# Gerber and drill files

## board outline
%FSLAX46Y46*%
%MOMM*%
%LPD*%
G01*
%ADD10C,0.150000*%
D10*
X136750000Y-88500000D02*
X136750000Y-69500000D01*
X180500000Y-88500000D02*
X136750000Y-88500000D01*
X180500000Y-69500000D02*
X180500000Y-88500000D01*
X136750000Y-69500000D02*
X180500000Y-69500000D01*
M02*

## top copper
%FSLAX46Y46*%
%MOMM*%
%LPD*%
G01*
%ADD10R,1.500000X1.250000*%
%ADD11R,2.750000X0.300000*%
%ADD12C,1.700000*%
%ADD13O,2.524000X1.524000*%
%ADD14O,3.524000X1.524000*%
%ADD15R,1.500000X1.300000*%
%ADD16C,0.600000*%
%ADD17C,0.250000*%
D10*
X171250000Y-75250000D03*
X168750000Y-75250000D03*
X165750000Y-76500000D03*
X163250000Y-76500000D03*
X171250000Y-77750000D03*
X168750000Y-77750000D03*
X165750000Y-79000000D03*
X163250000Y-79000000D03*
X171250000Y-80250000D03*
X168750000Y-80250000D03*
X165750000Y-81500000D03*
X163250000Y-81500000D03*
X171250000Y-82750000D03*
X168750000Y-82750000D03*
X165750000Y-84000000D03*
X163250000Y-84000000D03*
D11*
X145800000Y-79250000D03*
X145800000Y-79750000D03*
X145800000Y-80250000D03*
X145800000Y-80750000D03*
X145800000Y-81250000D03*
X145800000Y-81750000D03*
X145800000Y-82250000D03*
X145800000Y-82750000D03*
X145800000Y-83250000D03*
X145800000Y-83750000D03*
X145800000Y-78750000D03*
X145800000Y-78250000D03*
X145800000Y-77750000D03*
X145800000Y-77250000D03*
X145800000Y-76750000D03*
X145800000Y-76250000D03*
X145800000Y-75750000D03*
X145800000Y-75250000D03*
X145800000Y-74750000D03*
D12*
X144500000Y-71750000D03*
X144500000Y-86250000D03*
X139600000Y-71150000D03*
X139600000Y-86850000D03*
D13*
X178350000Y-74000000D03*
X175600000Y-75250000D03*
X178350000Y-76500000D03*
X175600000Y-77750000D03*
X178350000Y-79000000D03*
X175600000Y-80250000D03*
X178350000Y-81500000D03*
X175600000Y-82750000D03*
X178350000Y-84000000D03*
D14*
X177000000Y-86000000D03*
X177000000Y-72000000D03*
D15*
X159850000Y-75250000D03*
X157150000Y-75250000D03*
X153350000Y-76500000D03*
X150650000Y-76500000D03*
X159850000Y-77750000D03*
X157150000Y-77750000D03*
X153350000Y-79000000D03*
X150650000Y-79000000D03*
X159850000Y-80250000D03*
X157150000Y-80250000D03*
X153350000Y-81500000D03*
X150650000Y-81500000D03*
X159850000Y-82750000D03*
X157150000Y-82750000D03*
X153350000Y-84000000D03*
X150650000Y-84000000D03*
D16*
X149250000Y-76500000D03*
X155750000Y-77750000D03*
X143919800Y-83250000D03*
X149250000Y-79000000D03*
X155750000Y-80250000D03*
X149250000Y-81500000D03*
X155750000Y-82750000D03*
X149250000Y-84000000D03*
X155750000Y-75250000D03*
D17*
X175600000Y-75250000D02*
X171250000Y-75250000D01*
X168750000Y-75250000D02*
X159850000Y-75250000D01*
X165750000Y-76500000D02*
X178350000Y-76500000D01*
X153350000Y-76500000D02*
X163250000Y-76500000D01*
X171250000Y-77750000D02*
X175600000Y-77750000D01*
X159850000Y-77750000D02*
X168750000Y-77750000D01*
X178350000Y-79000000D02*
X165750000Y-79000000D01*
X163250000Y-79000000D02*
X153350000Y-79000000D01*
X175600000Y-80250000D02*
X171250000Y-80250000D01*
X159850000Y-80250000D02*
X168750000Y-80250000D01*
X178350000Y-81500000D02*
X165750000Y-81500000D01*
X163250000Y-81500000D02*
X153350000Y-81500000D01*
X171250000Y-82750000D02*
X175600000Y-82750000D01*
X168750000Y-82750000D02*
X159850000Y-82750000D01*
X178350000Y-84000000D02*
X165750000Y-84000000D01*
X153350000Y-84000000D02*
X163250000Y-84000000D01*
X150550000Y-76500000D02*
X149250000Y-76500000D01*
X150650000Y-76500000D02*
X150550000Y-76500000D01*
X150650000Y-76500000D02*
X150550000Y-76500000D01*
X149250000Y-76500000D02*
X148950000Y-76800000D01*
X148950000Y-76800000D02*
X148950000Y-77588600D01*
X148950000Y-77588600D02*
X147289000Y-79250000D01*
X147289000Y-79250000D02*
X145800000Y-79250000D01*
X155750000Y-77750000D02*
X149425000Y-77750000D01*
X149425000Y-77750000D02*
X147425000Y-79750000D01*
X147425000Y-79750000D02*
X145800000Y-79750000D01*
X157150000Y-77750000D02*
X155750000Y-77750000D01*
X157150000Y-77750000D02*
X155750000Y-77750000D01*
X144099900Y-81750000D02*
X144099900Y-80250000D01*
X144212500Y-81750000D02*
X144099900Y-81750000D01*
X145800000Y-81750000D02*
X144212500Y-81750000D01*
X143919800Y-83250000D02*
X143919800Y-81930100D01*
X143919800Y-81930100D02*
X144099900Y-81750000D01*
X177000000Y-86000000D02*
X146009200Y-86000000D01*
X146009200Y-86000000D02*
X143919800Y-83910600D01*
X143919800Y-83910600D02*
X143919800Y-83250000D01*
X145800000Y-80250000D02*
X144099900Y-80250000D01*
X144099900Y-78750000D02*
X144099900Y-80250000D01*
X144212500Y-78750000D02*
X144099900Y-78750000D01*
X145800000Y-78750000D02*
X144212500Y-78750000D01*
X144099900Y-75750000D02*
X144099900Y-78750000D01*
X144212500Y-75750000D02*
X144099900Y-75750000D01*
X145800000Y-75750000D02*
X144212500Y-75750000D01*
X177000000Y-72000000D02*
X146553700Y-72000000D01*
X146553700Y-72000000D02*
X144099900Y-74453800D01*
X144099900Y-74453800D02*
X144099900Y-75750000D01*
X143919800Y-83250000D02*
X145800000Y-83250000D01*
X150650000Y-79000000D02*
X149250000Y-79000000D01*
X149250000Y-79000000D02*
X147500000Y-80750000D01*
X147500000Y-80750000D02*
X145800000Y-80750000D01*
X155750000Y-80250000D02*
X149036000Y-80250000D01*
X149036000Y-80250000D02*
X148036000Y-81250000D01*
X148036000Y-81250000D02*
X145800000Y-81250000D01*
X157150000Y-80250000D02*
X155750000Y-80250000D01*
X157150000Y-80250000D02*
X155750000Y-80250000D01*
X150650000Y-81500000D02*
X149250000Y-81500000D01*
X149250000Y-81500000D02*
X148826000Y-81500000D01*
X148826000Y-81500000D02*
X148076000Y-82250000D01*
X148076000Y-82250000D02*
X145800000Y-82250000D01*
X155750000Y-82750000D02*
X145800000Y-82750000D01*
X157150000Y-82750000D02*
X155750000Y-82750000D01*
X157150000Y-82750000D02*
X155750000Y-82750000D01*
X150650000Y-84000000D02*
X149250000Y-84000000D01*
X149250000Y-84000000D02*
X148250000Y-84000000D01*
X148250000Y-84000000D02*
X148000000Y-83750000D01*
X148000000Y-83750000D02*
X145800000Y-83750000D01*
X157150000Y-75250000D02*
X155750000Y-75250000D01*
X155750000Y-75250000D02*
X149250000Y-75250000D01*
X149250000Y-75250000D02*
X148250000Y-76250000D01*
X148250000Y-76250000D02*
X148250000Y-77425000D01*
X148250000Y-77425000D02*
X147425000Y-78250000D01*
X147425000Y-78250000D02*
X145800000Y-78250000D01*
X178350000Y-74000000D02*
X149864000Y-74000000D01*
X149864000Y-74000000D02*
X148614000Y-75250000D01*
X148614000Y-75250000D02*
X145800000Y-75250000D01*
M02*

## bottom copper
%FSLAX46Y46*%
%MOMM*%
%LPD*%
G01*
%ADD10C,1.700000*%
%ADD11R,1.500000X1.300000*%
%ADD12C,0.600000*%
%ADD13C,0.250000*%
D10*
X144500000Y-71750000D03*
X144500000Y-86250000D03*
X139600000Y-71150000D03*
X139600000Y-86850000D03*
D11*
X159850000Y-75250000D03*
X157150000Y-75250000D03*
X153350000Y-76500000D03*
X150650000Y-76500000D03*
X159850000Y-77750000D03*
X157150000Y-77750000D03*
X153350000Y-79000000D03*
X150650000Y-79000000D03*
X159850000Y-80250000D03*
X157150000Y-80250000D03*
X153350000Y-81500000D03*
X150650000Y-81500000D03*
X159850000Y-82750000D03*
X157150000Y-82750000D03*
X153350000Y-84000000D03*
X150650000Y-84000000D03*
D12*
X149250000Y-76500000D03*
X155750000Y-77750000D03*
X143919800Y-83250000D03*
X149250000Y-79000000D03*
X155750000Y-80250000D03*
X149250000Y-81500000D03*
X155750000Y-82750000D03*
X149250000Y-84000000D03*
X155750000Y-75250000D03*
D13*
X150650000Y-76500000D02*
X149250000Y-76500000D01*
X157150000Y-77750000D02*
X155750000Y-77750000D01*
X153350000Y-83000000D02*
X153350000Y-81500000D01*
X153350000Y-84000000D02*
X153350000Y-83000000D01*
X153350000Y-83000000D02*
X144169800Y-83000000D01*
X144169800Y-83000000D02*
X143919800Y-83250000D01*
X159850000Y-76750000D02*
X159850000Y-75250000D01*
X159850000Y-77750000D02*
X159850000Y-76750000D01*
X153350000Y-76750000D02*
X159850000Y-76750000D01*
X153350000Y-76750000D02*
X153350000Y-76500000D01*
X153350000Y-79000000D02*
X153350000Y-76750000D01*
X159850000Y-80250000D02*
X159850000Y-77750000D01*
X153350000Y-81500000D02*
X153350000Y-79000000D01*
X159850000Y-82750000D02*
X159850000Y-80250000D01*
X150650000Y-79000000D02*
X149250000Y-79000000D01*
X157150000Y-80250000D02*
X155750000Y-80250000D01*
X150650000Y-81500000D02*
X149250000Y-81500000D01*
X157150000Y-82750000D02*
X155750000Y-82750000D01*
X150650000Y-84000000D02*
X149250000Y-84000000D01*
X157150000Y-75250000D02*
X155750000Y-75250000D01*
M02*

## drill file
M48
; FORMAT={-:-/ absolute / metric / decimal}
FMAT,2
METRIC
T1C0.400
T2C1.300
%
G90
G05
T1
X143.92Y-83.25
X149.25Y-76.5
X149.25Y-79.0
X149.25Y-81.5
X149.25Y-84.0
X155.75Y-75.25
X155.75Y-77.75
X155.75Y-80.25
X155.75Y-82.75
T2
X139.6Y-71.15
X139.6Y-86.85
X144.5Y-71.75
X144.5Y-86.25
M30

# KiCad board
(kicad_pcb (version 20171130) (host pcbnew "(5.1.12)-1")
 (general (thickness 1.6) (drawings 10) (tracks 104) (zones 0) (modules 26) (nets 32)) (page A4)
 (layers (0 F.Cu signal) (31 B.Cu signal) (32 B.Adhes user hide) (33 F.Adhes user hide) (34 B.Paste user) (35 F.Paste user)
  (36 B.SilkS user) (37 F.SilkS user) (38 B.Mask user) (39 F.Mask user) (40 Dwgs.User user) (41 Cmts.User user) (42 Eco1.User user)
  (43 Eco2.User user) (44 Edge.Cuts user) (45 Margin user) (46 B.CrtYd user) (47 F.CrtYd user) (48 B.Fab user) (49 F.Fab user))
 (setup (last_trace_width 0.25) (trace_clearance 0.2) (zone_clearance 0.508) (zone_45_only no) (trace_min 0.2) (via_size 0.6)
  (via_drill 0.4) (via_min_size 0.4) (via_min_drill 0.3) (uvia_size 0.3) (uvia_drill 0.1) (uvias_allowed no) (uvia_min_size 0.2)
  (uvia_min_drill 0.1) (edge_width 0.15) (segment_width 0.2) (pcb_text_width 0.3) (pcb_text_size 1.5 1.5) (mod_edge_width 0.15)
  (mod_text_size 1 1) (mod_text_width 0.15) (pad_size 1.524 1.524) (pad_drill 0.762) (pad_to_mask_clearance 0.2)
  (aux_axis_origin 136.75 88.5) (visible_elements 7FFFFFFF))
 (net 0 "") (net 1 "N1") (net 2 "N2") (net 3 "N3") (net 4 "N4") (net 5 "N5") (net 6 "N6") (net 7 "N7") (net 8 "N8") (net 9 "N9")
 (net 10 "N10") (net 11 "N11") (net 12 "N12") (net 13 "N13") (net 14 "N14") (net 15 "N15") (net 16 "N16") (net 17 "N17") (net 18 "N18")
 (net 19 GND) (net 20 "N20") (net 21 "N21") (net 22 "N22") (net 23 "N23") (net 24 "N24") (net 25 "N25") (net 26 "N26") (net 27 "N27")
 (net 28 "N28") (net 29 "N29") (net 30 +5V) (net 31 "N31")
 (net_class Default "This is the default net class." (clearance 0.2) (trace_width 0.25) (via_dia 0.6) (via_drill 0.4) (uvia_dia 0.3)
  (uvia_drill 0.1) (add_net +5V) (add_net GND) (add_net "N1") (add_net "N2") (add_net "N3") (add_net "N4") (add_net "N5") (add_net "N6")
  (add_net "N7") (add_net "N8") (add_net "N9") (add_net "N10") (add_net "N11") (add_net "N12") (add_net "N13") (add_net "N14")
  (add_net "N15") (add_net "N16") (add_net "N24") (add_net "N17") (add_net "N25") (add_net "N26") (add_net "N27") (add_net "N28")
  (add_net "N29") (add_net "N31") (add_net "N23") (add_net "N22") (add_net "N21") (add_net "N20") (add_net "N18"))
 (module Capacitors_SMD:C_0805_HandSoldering (layer F.Cu) (at 170 75.25 180)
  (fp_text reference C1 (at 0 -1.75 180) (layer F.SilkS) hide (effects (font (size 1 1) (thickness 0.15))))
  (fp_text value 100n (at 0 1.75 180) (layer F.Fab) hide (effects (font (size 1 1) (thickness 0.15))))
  (pad 1 smd rect (at -1.25 0 180) (size 1.5 1.25) (layers F.Cu F.Paste F.Mask) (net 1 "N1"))
  (pad 2 smd rect (at 1.25 0 180) (size 1.5 1.25) (layers F.Cu F.Paste F.Mask) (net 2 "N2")))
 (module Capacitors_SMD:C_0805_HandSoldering (layer F.Cu) (at 164.5 76.5 180)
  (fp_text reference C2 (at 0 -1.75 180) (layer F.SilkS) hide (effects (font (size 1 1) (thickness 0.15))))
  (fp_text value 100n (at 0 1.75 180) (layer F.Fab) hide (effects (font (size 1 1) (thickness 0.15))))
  (pad 1 smd rect (at -1.25 0 180) (size 1.5 1.25) (layers F.Cu F.Paste F.Mask) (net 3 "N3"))
  (pad 2 smd rect (at 1.25 0 180) (size 1.5 1.25) (layers F.Cu F.Paste F.Mask) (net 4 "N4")))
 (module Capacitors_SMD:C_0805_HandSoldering (layer F.Cu) (at 170 77.75 180)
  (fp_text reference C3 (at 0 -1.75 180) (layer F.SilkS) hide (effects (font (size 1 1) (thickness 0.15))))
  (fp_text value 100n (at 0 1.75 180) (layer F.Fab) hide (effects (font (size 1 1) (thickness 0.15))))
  (pad 1 smd rect (at -1.25 0 180) (size 1.5 1.25) (layers F.Cu F.Paste F.Mask) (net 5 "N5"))
  (pad 2 smd rect (at 1.25 0 180) (size 1.5 1.25) (layers F.Cu F.Paste F.Mask) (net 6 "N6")))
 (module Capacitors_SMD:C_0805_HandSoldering (layer F.Cu) (at 164.5 79 180)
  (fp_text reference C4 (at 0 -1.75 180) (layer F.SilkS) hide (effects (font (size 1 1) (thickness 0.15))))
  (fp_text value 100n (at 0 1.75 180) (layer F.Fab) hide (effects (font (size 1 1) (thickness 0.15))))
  (pad 1 smd rect (at -1.25 0 180) (size 1.5 1.25) (layers F.Cu F.Paste F.Mask) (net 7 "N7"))
  (pad 2 smd rect (at 1.25 0 180) (size 1.5 1.25) (layers F.Cu F.Paste F.Mask) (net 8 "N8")))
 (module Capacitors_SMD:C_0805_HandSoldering (layer F.Cu) (at 170 80.25 180)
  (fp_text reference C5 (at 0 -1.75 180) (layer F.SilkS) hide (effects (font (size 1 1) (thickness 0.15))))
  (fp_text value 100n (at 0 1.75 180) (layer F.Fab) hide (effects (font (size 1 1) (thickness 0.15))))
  (pad 1 smd rect (at -1.25 0 180) (size 1.5 1.25) (layers F.Cu F.Paste F.Mask) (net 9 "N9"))
  (pad 2 smd rect (at 1.25 0 180) (size 1.5 1.25) (layers F.Cu F.Paste F.Mask) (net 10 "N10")))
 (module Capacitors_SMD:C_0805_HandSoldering (layer F.Cu) (at 164.5 81.5 180)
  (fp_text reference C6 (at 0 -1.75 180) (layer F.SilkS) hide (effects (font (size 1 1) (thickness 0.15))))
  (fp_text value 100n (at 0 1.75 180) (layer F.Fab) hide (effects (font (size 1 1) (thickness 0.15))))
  (pad 1 smd rect (at -1.25 0 180) (size 1.5 1.25) (layers F.Cu F.Paste F.Mask) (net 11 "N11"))
  (pad 2 smd rect (at 1.25 0 180) (size 1.5 1.25) (layers F.Cu F.Paste F.Mask) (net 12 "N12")))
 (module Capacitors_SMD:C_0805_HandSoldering (layer F.Cu) (at 170 82.75 180)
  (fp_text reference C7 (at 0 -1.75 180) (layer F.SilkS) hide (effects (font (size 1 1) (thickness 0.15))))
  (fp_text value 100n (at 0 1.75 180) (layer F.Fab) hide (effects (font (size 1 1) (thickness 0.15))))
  (pad 1 smd rect (at -1.25 0 180) (size 1.5 1.25) (layers F.Cu F.Paste F.Mask) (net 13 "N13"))
  (pad 2 smd rect (at 1.25 0 180) (size 1.5 1.25) (layers F.Cu F.Paste F.Mask) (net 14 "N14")))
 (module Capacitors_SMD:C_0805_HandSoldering (layer F.Cu) (at 164.5 84 180)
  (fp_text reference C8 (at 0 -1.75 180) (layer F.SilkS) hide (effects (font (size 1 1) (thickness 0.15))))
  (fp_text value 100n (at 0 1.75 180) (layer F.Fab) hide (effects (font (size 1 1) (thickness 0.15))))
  (pad 1 smd rect (at -1.25 0 180) (size 1.5 1.25) (layers F.Cu F.Paste F.Mask) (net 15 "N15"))
  (pad 2 smd rect (at 1.25 0 180) (size 1.5 1.25) (layers F.Cu F.Paste F.Mask) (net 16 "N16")))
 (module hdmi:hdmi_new (layer F.Cu) (at 144.5 79 270)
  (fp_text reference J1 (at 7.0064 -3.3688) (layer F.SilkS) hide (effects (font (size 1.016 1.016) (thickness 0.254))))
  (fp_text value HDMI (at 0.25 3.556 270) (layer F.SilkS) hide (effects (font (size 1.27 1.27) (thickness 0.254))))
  (pad 10 smd rect (at 0.25 -1.3 270) (size 0.3 2.75) (layers F.Cu F.Paste F.Mask) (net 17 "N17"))
  (pad 9 smd rect (at 0.75 -1.3 270) (size 0.3 2.75) (layers F.Cu F.Paste F.Mask) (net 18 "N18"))
  (pad 8 smd rect (at 1.25 -1.3 270) (size 0.3 2.75) (layers F.Cu F.Paste F.Mask) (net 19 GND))
  (pad 7 smd rect (at 1.75 -1.3 270) (size 0.3 2.75) (layers F.Cu F.Paste F.Mask) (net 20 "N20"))
  (pad 6 smd rect (at 2.25 -1.3 270) (size 0.3 2.75) (layers F.Cu F.Paste F.Mask) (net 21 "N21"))
  (pad 5 smd rect (at 2.75 -1.3 270) (size 0.3 2.75) (layers F.Cu F.Paste F.Mask) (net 19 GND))
  (pad 4 smd rect (at 3.25 -1.3 270) (size 0.3 2.75) (layers F.Cu F.Paste F.Mask) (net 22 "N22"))
  (pad 3 smd rect (at 3.75 -1.3 270) (size 0.3 2.75) (layers F.Cu F.Paste F.Mask) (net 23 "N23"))
  (pad 2 smd rect (at 4.25 -1.3 270) (size 0.3 2.75) (layers F.Cu F.Paste F.Mask) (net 19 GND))
  (pad 1 smd rect (at 4.75 -1.3 270) (size 0.3 2.75) (layers F.Cu F.Paste F.Mask) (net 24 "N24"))
  (pad 11 smd rect (at -0.25 -1.3 270) (size 0.3 2.75) (layers F.Cu F.Paste F.Mask) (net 19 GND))
  (pad 12 smd rect (at -0.75 -1.3 270) (size 0.3 2.75) (layers F.Cu F.Paste F.Mask) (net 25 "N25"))
  (pad 13 smd rect (at -1.25 -1.3 270) (size 0.3 2.75) (layers F.Cu F.Paste F.Mask) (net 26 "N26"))
  (pad 14 smd rect (at -1.75 -1.3 270) (size 0.3 2.75) (layers F.Cu F.Paste F.Mask) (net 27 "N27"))
  (pad 15 smd rect (at -2.25 -1.3 270) (size 0.3 2.75) (layers F.Cu F.Paste F.Mask) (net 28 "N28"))
  (pad 16 smd rect (at -2.75 -1.3 270) (size 0.3 2.75) (layers F.Cu F.Paste F.Mask) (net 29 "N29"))
  (pad 17 smd rect (at -3.25 -1.3 270) (size 0.3 2.75) (layers F.Cu F.Paste F.Mask) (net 19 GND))
  (pad 18 smd rect (at -3.75 -1.3 270) (size 0.3 2.75) (layers F.Cu F.Paste F.Mask) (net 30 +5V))
  (pad 19 smd rect (at -4.25 -1.3 270) (size 0.3 2.75) (layers F.Cu F.Paste F.Mask) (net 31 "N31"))
  (pad 0 thru_hole circle (at -7.25 0 270) (size 1.7 1.7) (drill 1.3) (layers *.Cu *.Mask F.SilkS))
  (pad 0 thru_hole circle (at 7.25 0 270) (size 1.7 1.7) (drill 1.3) (layers *.Cu *.Mask F.SilkS))
  (pad 0 thru_hole circle (at -7.85 4.9 270) (size 1.7 1.7) (drill 1.3) (layers *.Cu *.Mask F.SilkS))
  (pad 0 thru_hole circle (at 7.85 4.9 270) (size 1.7 1.7) (drill 1.3) (layers *.Cu *.Mask F.SilkS)))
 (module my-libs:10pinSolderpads (layer F.Cu) (at 177 79 270)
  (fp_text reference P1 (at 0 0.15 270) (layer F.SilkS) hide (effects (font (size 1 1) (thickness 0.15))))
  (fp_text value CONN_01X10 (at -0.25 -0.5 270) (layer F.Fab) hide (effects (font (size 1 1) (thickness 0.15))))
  (pad 1 smd oval (at -5 -1.35 270) (size 1.524 2.524) (layers F.Cu F.Paste F.Mask) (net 30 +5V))
  (pad 2 smd oval (at -3.75 1.4 270) (size 1.524 2.524) (layers F.Cu F.Paste F.Mask) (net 1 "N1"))
  (pad 3 smd oval (at -2.5 -1.35 270) (size 1.524 2.524) (layers F.Cu F.Paste F.Mask) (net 3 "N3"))
  (pad 4 smd oval (at -1.25 1.4 270) (size 1.524 2.524) (layers F.Cu F.Paste F.Mask) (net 5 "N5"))
  (pad 5 smd oval (at 0 -1.35 270) (size 1.524 2.524) (layers F.Cu F.Paste F.Mask) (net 7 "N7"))
  (pad 6 smd oval (at 1.25 1.4 270) (size 1.524 2.524) (layers F.Cu F.Paste F.Mask) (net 9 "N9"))
  (pad 7 smd oval (at 2.5 -1.35 270) (size 1.524 2.524) (layers F.Cu F.Paste F.Mask) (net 11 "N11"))
  (pad 8 smd oval (at 3.75 1.4 270) (size 1.524 2.524) (layers F.Cu F.Paste F.Mask) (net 13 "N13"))
  (pad 9 smd oval (at 5 -1.35 270) (size 1.524 2.524) (layers F.Cu F.Paste F.Mask) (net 15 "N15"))
  (pad 10 smd oval (at 7 0 90) (size 1.524 3.524) (layers F.Cu F.Paste F.Mask) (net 19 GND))
  (pad 10 smd oval (at -7 0 90) (size 1.524 3.524) (layers F.Cu F.Paste F.Mask) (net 19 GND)))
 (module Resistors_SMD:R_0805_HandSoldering (layer F.Cu) (at 158.5 75.25 180)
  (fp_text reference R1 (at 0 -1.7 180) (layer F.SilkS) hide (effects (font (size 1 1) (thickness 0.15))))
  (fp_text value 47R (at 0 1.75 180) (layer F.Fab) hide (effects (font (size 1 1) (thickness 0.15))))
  (pad 1 smd rect (at -1.35 0 180) (size 1.5 1.3) (layers F.Cu F.Paste F.Mask) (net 2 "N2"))
  (pad 2 smd rect (at 1.35 0 180) (size 1.5 1.3) (layers F.Cu F.Paste F.Mask) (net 25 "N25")))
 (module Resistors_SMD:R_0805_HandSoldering (layer F.Cu) (at 152 76.5 180)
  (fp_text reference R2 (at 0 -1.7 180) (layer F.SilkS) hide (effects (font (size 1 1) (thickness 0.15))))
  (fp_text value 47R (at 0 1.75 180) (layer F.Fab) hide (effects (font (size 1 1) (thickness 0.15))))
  (pad 1 smd rect (at -1.35 0 180) (size 1.5 1.3) (layers F.Cu F.Paste F.Mask) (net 4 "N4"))
  (pad 2 smd rect (at 1.35 0 180) (size 1.5 1.3) (layers F.Cu F.Paste F.Mask) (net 17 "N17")))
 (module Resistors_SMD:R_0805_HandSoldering (layer B.Cu) (at 158.5 75.25 180)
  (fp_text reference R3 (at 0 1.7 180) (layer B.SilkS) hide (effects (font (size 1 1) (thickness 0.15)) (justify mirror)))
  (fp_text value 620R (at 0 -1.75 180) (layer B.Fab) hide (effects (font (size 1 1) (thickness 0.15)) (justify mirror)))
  (pad 1 smd rect (at -1.35 0 180) (size 1.5 1.3) (layers B.Cu B.Paste B.Mask) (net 19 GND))
  (pad 2 smd rect (at 1.35 0 180) (size 1.5 1.3) (layers B.Cu B.Paste B.Mask) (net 25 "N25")))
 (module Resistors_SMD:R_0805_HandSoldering (layer B.Cu) (at 152 76.5 180)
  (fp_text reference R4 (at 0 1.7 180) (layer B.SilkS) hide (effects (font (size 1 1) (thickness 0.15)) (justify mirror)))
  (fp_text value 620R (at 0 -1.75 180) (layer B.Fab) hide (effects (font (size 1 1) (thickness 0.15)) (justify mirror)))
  (pad 1 smd rect (at -1.35 0 180) (size 1.5 1.3) (layers B.Cu B.Paste B.Mask) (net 19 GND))
  (pad 2 smd rect (at 1.35 0 180) (size 1.5 1.3) (layers B.Cu B.Paste B.Mask) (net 17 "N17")))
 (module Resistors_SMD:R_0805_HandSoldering (layer F.Cu) (at 158.5 77.75 180)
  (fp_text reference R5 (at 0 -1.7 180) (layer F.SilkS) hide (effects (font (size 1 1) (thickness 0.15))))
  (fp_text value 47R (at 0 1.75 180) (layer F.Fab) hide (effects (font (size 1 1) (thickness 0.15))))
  (pad 1 smd rect (at -1.35 0 180) (size 1.5 1.3) (layers F.Cu F.Paste F.Mask) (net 6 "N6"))
  (pad 2 smd rect (at 1.35 0 180) (size 1.5 1.3) (layers F.Cu F.Paste F.Mask) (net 18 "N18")))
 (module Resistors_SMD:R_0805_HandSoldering (layer F.Cu) (at 152 79 180)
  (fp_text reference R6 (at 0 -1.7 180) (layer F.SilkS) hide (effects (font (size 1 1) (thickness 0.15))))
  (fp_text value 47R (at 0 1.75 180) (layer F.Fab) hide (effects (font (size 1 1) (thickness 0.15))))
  (pad 1 smd rect (at -1.35 0 180) (size 1.5 1.3) (layers F.Cu F.Paste F.Mask) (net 8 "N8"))
  (pad 2 smd rect (at 1.35 0 180) (size 1.5 1.3) (layers F.Cu F.Paste F.Mask) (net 20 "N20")))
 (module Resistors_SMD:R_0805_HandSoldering (layer B.Cu) (at 158.5 77.75 180)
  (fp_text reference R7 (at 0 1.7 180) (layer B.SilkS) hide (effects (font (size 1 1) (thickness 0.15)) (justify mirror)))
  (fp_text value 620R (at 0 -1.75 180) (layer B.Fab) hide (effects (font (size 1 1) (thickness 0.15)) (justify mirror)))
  (pad 1 smd rect (at -1.35 0 180) (size 1.5 1.3) (layers B.Cu B.Paste B.Mask) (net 19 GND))
  (pad 2 smd rect (at 1.35 0 180) (size 1.5 1.3) (layers B.Cu B.Paste B.Mask) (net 18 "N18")))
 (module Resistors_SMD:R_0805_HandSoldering (layer B.Cu) (at 152 79 180)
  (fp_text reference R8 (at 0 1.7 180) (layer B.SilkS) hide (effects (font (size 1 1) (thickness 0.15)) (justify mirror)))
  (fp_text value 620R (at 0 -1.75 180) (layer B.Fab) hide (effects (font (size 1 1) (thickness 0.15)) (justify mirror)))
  (pad 1 smd rect (at -1.35 0 180) (size 1.5 1.3) (layers B.Cu B.Paste B.Mask) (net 19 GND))
  (pad 2 smd rect (at 1.35 0 180) (size 1.5 1.3) (layers B.Cu B.Paste B.Mask) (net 20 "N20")))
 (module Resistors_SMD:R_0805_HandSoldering (layer F.Cu) (at 158.5 80.25 180)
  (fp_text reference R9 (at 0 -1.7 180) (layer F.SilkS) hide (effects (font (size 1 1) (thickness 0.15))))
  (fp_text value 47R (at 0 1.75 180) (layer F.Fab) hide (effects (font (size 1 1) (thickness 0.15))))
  (pad 1 smd rect (at -1.35 0 180) (size 1.5 1.3) (layers F.Cu F.Paste F.Mask) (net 10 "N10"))
  (pad 2 smd rect (at 1.35 0 180) (size 1.5 1.3) (layers F.Cu F.Paste F.Mask) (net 21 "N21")))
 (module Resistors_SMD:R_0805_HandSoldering (layer F.Cu) (at 152 81.5 180)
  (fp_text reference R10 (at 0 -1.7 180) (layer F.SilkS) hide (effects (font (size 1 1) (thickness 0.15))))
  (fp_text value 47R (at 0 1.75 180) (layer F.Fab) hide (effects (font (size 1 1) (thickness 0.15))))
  (pad 1 smd rect (at -1.35 0 180) (size 1.5 1.3) (layers F.Cu F.Paste F.Mask) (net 12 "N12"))
  (pad 2 smd rect (at 1.35 0 180) (size 1.5 1.3) (layers F.Cu F.Paste F.Mask) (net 22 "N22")))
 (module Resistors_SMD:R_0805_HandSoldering (layer B.Cu) (at 158.5 80.25 180)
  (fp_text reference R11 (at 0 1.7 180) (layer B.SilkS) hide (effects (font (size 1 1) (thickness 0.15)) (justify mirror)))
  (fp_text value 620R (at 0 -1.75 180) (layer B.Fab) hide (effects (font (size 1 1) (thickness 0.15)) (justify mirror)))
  (pad 1 smd rect (at -1.35 0 180) (size 1.5 1.3) (layers B.Cu B.Paste B.Mask) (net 19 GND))
  (pad 2 smd rect (at 1.35 0 180) (size 1.5 1.3) (layers B.Cu B.Paste B.Mask) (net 21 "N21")))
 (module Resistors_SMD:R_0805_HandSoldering (layer B.Cu) (at 152 81.5 180)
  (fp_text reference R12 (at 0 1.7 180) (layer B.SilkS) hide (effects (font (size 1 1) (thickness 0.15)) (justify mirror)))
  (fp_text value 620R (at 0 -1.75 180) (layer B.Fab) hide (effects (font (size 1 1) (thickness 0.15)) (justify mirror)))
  (pad 1 smd rect (at -1.35 0 180) (size 1.5 1.3) (layers B.Cu B.Paste B.Mask) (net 19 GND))
  (pad 2 smd rect (at 1.35 0 180) (size 1.5 1.3) (layers B.Cu B.Paste B.Mask) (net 22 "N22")))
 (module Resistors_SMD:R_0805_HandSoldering (layer F.Cu) (at 158.5 82.75 180)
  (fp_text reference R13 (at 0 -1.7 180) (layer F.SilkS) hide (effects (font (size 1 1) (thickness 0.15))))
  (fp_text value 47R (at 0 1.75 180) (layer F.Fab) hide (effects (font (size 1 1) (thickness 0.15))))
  (pad 1 smd rect (at -1.35 0 180) (size 1.5 1.3) (layers F.Cu F.Paste F.Mask) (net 14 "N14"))
  (pad 2 smd rect (at 1.35 0 180) (size 1.5 1.3) (layers F.Cu F.Paste F.Mask) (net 23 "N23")))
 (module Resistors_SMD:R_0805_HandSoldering (layer F.Cu) (at 152 84 180)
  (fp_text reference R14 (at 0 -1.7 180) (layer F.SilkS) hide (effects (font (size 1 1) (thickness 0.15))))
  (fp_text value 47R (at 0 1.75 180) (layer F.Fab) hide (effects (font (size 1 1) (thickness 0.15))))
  (pad 1 smd rect (at -1.35 0 180) (size 1.5 1.3) (layers F.Cu F.Paste F.Mask) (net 16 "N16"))
  (pad 2 smd rect (at 1.35 0 180) (size 1.5 1.3) (layers F.Cu F.Paste F.Mask) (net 24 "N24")))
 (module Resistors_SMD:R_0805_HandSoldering (layer B.Cu) (at 158.5 82.75 180)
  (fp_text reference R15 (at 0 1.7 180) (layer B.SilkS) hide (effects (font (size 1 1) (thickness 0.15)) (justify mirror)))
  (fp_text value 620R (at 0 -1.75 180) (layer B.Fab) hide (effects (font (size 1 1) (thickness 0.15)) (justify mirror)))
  (pad 1 smd rect (at -1.35 0 180) (size 1.5 1.3) (layers B.Cu B.Paste B.Mask) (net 19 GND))
  (pad 2 smd rect (at 1.35 0 180) (size 1.5 1.3) (layers B.Cu B.Paste B.Mask) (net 23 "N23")))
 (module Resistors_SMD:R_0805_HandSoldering (layer B.Cu) (at 152 84 180)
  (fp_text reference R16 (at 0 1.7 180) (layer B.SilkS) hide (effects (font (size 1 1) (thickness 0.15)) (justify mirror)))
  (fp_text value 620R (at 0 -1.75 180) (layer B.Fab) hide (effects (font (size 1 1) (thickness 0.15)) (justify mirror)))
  (pad 1 smd rect (at -1.35 0 180) (size 1.5 1.3) (layers B.Cu B.Paste B.Mask) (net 19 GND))
  (pad 2 smd rect (at 1.35 0 180) (size 1.5 1.3) (layers B.Cu B.Paste B.Mask) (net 24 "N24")))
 (gr_line (start 136.75 88.5) (end 136.75 69.5) (layer Edge.Cuts) (width 0.15))
 (gr_line (start 180.5 88.5) (end 136.75 88.5) (layer Edge.Cuts) (width 0.15))
 (gr_line (start 180.5 69.5) (end 180.5 88.5) (layer Edge.Cuts) (width 0.15))
 (gr_line (start 136.75 69.5) (end 180.5 69.5) (layer Edge.Cuts) (width 0.15))
 (segment (start 175.6 75.25) (end 171.25 75.25) (width 0.25) (layer F.Cu) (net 1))
 (segment (start 168.75 75.25) (end 159.85 75.25) (width 0.25) (layer F.Cu) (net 2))
 (segment (start 165.75 76.5) (end 178.35 76.5) (width 0.25) (layer F.Cu) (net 3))
 (segment (start 153.35 76.5) (end 163.25 76.5) (width 0.25) (layer F.Cu) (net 4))
 (segment (start 171.25 77.75) (end 175.6 77.75) (width 0.25) (layer F.Cu) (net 5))
 (segment (start 159.85 77.75) (end 168.75 77.75) (width 0.25) (layer F.Cu) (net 6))
 (segment (start 178.35 79) (end 165.75 79) (width 0.25) (layer F.Cu) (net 7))
 (segment (start 163.25 79) (end 153.35 79) (width 0.25) (layer F.Cu) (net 8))
 (segment (start 175.6 80.25) (end 171.25 80.25) (width 0.25) (layer F.Cu) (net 9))
 (segment (start 159.85 80.25) (end 168.75 80.25) (width 0.25) (layer F.Cu) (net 10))
 (segment (start 178.35 81.5) (end 165.75 81.5) (width 0.25) (layer F.Cu) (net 11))
 (segment (start 163.25 81.5) (end 153.35 81.5) (width 0.25) (layer F.Cu) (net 12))
 (segment (start 171.25 82.75) (end 175.6 82.75) (width 0.25) (layer F.Cu) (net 13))
 (segment (start 168.75 82.75) (end 159.85 82.75) (width 0.25) (layer F.Cu) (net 14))
 (segment (start 178.35 84) (end 165.75 84) (width 0.25) (layer F.Cu) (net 15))
 (segment (start 153.35 84) (end 163.25 84) (width 0.25) (layer F.Cu) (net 16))
 (segment (start 150.55 76.5) (end 149.25 76.5) (width 0.25) (layer F.Cu) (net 17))
 (segment (start 150.65 76.5) (end 150.55 76.5) (width 0.25) (layer F.Cu) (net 17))
 (segment (start 150.65 76.5) (end 150.55 76.5) (width 0.25) (layer F.Cu) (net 17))
 (segment (start 150.65 76.5) (end 149.25 76.5) (width 0.25) (layer B.Cu) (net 17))
 (segment (start 149.25 76.5) (end 148.95 76.8) (width 0.25) (layer F.Cu) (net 17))
 (segment (start 148.95 76.8) (end 148.95 77.5886) (width 0.25) (layer F.Cu) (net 17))
 (segment (start 148.95 77.5886) (end 147.289 79.25) (width 0.25) (layer F.Cu) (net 17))
 (segment (start 147.289 79.25) (end 145.8 79.25) (width 0.25) (layer F.Cu) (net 17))
 (via (at 149.25 76.5) (size 0.6) (layers F.Cu B.Cu) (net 17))
 (segment (start 155.75 77.75) (end 149.425 77.75) (width 0.25) (layer F.Cu) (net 18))
 (segment (start 149.425 77.75) (end 147.425 79.75) (width 0.25) (layer F.Cu) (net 18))
 (segment (start 147.425 79.75) (end 145.8 79.75) (width 0.25) (layer F.Cu) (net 18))
 (segment (start 157.15 77.75) (end 155.75 77.75) (width 0.25) (layer F.Cu) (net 18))
 (segment (start 157.15 77.75) (end 155.75 77.75) (width 0.25) (layer B.Cu) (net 18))
 (segment (start 157.15 77.75) (end 155.75 77.75) (width 0.25) (layer F.Cu) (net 18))
 (via (at 155.75 77.75) (size 0.6) (layers F.Cu B.Cu) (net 18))
 (segment (start 144.0999 81.75) (end 144.0999 80.25) (width 0.25) (layer F.Cu) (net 19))
 (segment (start 144.2125 81.75) (end 144.0999 81.75) (width 0.25) (layer F.Cu) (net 19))
 (segment (start 145.8 81.75) (end 144.2125 81.75) (width 0.25) (layer F.Cu) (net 19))
 (segment (start 143.9198 83.25) (end 143.9198 81.9301) (width 0.25) (layer F.Cu) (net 19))
 (segment (start 143.9198 81.9301) (end 144.0999 81.75) (width 0.25) (layer F.Cu) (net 19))
 (segment (start 177 86) (end 146.0092 86) (width 0.25) (layer F.Cu) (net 19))
 (segment (start 146.0092 86) (end 143.9198 83.9106) (width 0.25) (layer F.Cu) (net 19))
 (segment (start 143.9198 83.9106) (end 143.9198 83.25) (width 0.25) (layer F.Cu) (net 19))
 (segment (start 145.8 80.25) (end 144.0999 80.25) (width 0.25) (layer F.Cu) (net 19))
 (segment (start 144.0999 78.75) (end 144.0999 80.25) (width 0.25) (layer F.Cu) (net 19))
 (segment (start 144.2125 78.75) (end 144.0999 78.75) (width 0.25) (layer F.Cu) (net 19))
 (segment (start 145.8 78.75) (end 144.2125 78.75) (width 0.25) (layer F.Cu) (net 19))
 (segment (start 144.0999 75.75) (end 144.0999 78.75) (width 0.25) (layer F.Cu) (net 19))
 (segment (start 144.2125 75.75) (end 144.0999 75.75) (width 0.25) (layer F.Cu) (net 19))
 (segment (start 145.8 75.75) (end 144.2125 75.75) (width 0.25) (layer F.Cu) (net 19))
 (segment (start 177 72) (end 146.5537 72) (width 0.25) (layer F.Cu) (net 19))
 (segment (start 146.5537 72) (end 144.0999 74.4538) (width 0.25) (layer F.Cu) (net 19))
 (segment (start 144.0999 74.4538) (end 144.0999 75.75) (width 0.25) (layer F.Cu) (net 19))
 (segment (start 153.35 83) (end 153.35 81.5) (width 0.25) (layer B.Cu) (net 19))
 (segment (start 153.35 84) (end 153.35 83) (width 0.25) (layer B.Cu) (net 19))
 (segment (start 153.35 83) (end 144.1698 83) (width 0.25) (layer B.Cu) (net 19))
 (segment (start 144.1698 83) (end 143.9198 83.25) (width 0.25) (layer B.Cu) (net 19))
 (segment (start 143.9198 83.25) (end 145.8 83.25) (width 0.25) (layer F.Cu) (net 19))
 (segment (start 159.85 76.75) (end 159.85 75.25) (width 0.25) (layer B.Cu) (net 19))
 (segment (start 159.85 77.75) (end 159.85 76.75) (width 0.25) (layer B.Cu) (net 19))
 (segment (start 153.35 76.75) (end 159.85 76.75) (width 0.25) (layer B.Cu) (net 19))
 (segment (start 153.35 76.75) (end 153.35 76.5) (width 0.25) (layer B.Cu) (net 19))
 (segment (start 153.35 79) (end 153.35 76.75) (width 0.25) (layer B.Cu) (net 19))
 (segment (start 159.85 80.25) (end 159.85 77.75) (width 0.25) (layer B.Cu) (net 19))
 (segment (start 153.35 81.5) (end 153.35 79) (width 0.25) (layer B.Cu) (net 19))
 (segment (start 159.85 82.75) (end 159.85 80.25) (width 0.25) (layer B.Cu) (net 19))
 (via (at 143.9198 83.25) (size 0.6) (layers F.Cu B.Cu) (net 19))
 (segment (start 150.65 79) (end 149.25 79) (width 0.25) (layer F.Cu) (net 20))
 (segment (start 150.65 79) (end 149.25 79) (width 0.25) (layer B.Cu) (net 20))
 (segment (start 149.25 79) (end 147.5 80.75) (width 0.25) (layer F.Cu) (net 20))
 (segment (start 147.5 80.75) (end 145.8 80.75) (width 0.25) (layer F.Cu) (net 20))
 (via (at 149.25 79) (size 0.6) (layers F.Cu B.Cu) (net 20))
 (segment (start 155.75 80.25) (end 149.036 80.25) (width 0.25) (layer F.Cu) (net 21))
 (segment (start 149.036 80.25) (end 148.036 81.25) (width 0.25) (layer F.Cu) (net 21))
 (segment (start 148.036 81.25) (end 145.8 81.25) (width 0.25) (layer F.Cu) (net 21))
 (segment (start 157.15 80.25) (end 155.75 80.25) (width 0.25) (layer F.Cu) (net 21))
 (segment (start 157.15 80.25) (end 155.75 80.25) (width 0.25) (layer B.Cu) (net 21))
 (segment (start 157.15 80.25) (end 155.75 80.25) (width 0.25) (layer F.Cu) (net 21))
 (via (at 155.75 80.25) (size 0.6) (layers F.Cu B.Cu) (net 21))
 (segment (start 150.65 81.5) (end 149.25 81.5) (width 0.25) (layer F.Cu) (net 22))
 (segment (start 150.65 81.5) (end 149.25 81.5) (width 0.25) (layer B.Cu) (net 22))
 (segment (start 149.25 81.5) (end 148.826 81.5) (width 0.25) (layer F.Cu) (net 22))
 (segment (start 148.826 81.5) (end 148.076 82.25) (width 0.25) (layer F.Cu) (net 22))
 (segment (start 148.076 82.25) (end 145.8 82.25) (width 0.25) (layer F.Cu) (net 22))
 (via (at 149.25 81.5) (size 0.6) (layers F.Cu B.Cu) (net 22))
 (segment (start 155.75 82.75) (end 145.8 82.75) (width 0.25) (layer F.Cu) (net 23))
 (segment (start 157.15 82.75) (end 155.75 82.75) (width 0.25) (layer F.Cu) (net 23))
 (segment (start 157.15 82.75) (end 155.75 82.75) (width 0.25) (layer B.Cu) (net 23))
 (segment (start 157.15 82.75) (end 155.75 82.75) (width 0.25) (layer F.Cu) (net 23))
 (via (at 155.75 82.75) (size 0.6) (layers F.Cu B.Cu) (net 23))
 (segment (start 150.65 84) (end 149.25 84) (width 0.25) (layer B.Cu) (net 24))
 (segment (start 150.65 84) (end 149.25 84) (width 0.25) (layer F.Cu) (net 24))
 (segment (start 149.25 84) (end 148.25 84) (width 0.25) (layer F.Cu) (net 24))
 (segment (start 148.25 84) (end 148 83.75) (width 0.25) (layer F.Cu) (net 24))
 (segment (start 148 83.75) (end 145.8 83.75) (width 0.25) (layer F.Cu) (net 24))
 (via (at 149.25 84) (size 0.6) (layers F.Cu B.Cu) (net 24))
 (segment (start 157.15 75.25) (end 155.75 75.25) (width 0.25) (layer B.Cu) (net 25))
 (segment (start 157.15 75.25) (end 155.75 75.25) (width 0.25) (layer F.Cu) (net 25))
 (segment (start 155.75 75.25) (end 149.25 75.25) (width 0.25) (layer F.Cu) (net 25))
 (segment (start 149.25 75.25) (end 148.25 76.25) (width 0.25) (layer F.Cu) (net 25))
 (segment (start 148.25 76.25) (end 148.25 77.425) (width 0.25) (layer F.Cu) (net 25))
 (segment (start 148.25 77.425) (end 147.425 78.25) (width 0.25) (layer F.Cu) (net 25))
 (segment (start 147.425 78.25) (end 145.8 78.25) (width 0.25) (layer F.Cu) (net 25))
 (via (at 155.75 75.25) (size 0.6) (layers F.Cu B.Cu) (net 25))
 (segment (start 178.35 74) (end 149.864 74) (width 0.25) (layer F.Cu) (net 30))
 (segment (start 149.864 74) (end 148.614 75.25) (width 0.25) (layer F.Cu) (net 30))
 (segment (start 148.614 75.25) (end 145.8 75.25) (width 0.25) (layer F.Cu) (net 30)))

